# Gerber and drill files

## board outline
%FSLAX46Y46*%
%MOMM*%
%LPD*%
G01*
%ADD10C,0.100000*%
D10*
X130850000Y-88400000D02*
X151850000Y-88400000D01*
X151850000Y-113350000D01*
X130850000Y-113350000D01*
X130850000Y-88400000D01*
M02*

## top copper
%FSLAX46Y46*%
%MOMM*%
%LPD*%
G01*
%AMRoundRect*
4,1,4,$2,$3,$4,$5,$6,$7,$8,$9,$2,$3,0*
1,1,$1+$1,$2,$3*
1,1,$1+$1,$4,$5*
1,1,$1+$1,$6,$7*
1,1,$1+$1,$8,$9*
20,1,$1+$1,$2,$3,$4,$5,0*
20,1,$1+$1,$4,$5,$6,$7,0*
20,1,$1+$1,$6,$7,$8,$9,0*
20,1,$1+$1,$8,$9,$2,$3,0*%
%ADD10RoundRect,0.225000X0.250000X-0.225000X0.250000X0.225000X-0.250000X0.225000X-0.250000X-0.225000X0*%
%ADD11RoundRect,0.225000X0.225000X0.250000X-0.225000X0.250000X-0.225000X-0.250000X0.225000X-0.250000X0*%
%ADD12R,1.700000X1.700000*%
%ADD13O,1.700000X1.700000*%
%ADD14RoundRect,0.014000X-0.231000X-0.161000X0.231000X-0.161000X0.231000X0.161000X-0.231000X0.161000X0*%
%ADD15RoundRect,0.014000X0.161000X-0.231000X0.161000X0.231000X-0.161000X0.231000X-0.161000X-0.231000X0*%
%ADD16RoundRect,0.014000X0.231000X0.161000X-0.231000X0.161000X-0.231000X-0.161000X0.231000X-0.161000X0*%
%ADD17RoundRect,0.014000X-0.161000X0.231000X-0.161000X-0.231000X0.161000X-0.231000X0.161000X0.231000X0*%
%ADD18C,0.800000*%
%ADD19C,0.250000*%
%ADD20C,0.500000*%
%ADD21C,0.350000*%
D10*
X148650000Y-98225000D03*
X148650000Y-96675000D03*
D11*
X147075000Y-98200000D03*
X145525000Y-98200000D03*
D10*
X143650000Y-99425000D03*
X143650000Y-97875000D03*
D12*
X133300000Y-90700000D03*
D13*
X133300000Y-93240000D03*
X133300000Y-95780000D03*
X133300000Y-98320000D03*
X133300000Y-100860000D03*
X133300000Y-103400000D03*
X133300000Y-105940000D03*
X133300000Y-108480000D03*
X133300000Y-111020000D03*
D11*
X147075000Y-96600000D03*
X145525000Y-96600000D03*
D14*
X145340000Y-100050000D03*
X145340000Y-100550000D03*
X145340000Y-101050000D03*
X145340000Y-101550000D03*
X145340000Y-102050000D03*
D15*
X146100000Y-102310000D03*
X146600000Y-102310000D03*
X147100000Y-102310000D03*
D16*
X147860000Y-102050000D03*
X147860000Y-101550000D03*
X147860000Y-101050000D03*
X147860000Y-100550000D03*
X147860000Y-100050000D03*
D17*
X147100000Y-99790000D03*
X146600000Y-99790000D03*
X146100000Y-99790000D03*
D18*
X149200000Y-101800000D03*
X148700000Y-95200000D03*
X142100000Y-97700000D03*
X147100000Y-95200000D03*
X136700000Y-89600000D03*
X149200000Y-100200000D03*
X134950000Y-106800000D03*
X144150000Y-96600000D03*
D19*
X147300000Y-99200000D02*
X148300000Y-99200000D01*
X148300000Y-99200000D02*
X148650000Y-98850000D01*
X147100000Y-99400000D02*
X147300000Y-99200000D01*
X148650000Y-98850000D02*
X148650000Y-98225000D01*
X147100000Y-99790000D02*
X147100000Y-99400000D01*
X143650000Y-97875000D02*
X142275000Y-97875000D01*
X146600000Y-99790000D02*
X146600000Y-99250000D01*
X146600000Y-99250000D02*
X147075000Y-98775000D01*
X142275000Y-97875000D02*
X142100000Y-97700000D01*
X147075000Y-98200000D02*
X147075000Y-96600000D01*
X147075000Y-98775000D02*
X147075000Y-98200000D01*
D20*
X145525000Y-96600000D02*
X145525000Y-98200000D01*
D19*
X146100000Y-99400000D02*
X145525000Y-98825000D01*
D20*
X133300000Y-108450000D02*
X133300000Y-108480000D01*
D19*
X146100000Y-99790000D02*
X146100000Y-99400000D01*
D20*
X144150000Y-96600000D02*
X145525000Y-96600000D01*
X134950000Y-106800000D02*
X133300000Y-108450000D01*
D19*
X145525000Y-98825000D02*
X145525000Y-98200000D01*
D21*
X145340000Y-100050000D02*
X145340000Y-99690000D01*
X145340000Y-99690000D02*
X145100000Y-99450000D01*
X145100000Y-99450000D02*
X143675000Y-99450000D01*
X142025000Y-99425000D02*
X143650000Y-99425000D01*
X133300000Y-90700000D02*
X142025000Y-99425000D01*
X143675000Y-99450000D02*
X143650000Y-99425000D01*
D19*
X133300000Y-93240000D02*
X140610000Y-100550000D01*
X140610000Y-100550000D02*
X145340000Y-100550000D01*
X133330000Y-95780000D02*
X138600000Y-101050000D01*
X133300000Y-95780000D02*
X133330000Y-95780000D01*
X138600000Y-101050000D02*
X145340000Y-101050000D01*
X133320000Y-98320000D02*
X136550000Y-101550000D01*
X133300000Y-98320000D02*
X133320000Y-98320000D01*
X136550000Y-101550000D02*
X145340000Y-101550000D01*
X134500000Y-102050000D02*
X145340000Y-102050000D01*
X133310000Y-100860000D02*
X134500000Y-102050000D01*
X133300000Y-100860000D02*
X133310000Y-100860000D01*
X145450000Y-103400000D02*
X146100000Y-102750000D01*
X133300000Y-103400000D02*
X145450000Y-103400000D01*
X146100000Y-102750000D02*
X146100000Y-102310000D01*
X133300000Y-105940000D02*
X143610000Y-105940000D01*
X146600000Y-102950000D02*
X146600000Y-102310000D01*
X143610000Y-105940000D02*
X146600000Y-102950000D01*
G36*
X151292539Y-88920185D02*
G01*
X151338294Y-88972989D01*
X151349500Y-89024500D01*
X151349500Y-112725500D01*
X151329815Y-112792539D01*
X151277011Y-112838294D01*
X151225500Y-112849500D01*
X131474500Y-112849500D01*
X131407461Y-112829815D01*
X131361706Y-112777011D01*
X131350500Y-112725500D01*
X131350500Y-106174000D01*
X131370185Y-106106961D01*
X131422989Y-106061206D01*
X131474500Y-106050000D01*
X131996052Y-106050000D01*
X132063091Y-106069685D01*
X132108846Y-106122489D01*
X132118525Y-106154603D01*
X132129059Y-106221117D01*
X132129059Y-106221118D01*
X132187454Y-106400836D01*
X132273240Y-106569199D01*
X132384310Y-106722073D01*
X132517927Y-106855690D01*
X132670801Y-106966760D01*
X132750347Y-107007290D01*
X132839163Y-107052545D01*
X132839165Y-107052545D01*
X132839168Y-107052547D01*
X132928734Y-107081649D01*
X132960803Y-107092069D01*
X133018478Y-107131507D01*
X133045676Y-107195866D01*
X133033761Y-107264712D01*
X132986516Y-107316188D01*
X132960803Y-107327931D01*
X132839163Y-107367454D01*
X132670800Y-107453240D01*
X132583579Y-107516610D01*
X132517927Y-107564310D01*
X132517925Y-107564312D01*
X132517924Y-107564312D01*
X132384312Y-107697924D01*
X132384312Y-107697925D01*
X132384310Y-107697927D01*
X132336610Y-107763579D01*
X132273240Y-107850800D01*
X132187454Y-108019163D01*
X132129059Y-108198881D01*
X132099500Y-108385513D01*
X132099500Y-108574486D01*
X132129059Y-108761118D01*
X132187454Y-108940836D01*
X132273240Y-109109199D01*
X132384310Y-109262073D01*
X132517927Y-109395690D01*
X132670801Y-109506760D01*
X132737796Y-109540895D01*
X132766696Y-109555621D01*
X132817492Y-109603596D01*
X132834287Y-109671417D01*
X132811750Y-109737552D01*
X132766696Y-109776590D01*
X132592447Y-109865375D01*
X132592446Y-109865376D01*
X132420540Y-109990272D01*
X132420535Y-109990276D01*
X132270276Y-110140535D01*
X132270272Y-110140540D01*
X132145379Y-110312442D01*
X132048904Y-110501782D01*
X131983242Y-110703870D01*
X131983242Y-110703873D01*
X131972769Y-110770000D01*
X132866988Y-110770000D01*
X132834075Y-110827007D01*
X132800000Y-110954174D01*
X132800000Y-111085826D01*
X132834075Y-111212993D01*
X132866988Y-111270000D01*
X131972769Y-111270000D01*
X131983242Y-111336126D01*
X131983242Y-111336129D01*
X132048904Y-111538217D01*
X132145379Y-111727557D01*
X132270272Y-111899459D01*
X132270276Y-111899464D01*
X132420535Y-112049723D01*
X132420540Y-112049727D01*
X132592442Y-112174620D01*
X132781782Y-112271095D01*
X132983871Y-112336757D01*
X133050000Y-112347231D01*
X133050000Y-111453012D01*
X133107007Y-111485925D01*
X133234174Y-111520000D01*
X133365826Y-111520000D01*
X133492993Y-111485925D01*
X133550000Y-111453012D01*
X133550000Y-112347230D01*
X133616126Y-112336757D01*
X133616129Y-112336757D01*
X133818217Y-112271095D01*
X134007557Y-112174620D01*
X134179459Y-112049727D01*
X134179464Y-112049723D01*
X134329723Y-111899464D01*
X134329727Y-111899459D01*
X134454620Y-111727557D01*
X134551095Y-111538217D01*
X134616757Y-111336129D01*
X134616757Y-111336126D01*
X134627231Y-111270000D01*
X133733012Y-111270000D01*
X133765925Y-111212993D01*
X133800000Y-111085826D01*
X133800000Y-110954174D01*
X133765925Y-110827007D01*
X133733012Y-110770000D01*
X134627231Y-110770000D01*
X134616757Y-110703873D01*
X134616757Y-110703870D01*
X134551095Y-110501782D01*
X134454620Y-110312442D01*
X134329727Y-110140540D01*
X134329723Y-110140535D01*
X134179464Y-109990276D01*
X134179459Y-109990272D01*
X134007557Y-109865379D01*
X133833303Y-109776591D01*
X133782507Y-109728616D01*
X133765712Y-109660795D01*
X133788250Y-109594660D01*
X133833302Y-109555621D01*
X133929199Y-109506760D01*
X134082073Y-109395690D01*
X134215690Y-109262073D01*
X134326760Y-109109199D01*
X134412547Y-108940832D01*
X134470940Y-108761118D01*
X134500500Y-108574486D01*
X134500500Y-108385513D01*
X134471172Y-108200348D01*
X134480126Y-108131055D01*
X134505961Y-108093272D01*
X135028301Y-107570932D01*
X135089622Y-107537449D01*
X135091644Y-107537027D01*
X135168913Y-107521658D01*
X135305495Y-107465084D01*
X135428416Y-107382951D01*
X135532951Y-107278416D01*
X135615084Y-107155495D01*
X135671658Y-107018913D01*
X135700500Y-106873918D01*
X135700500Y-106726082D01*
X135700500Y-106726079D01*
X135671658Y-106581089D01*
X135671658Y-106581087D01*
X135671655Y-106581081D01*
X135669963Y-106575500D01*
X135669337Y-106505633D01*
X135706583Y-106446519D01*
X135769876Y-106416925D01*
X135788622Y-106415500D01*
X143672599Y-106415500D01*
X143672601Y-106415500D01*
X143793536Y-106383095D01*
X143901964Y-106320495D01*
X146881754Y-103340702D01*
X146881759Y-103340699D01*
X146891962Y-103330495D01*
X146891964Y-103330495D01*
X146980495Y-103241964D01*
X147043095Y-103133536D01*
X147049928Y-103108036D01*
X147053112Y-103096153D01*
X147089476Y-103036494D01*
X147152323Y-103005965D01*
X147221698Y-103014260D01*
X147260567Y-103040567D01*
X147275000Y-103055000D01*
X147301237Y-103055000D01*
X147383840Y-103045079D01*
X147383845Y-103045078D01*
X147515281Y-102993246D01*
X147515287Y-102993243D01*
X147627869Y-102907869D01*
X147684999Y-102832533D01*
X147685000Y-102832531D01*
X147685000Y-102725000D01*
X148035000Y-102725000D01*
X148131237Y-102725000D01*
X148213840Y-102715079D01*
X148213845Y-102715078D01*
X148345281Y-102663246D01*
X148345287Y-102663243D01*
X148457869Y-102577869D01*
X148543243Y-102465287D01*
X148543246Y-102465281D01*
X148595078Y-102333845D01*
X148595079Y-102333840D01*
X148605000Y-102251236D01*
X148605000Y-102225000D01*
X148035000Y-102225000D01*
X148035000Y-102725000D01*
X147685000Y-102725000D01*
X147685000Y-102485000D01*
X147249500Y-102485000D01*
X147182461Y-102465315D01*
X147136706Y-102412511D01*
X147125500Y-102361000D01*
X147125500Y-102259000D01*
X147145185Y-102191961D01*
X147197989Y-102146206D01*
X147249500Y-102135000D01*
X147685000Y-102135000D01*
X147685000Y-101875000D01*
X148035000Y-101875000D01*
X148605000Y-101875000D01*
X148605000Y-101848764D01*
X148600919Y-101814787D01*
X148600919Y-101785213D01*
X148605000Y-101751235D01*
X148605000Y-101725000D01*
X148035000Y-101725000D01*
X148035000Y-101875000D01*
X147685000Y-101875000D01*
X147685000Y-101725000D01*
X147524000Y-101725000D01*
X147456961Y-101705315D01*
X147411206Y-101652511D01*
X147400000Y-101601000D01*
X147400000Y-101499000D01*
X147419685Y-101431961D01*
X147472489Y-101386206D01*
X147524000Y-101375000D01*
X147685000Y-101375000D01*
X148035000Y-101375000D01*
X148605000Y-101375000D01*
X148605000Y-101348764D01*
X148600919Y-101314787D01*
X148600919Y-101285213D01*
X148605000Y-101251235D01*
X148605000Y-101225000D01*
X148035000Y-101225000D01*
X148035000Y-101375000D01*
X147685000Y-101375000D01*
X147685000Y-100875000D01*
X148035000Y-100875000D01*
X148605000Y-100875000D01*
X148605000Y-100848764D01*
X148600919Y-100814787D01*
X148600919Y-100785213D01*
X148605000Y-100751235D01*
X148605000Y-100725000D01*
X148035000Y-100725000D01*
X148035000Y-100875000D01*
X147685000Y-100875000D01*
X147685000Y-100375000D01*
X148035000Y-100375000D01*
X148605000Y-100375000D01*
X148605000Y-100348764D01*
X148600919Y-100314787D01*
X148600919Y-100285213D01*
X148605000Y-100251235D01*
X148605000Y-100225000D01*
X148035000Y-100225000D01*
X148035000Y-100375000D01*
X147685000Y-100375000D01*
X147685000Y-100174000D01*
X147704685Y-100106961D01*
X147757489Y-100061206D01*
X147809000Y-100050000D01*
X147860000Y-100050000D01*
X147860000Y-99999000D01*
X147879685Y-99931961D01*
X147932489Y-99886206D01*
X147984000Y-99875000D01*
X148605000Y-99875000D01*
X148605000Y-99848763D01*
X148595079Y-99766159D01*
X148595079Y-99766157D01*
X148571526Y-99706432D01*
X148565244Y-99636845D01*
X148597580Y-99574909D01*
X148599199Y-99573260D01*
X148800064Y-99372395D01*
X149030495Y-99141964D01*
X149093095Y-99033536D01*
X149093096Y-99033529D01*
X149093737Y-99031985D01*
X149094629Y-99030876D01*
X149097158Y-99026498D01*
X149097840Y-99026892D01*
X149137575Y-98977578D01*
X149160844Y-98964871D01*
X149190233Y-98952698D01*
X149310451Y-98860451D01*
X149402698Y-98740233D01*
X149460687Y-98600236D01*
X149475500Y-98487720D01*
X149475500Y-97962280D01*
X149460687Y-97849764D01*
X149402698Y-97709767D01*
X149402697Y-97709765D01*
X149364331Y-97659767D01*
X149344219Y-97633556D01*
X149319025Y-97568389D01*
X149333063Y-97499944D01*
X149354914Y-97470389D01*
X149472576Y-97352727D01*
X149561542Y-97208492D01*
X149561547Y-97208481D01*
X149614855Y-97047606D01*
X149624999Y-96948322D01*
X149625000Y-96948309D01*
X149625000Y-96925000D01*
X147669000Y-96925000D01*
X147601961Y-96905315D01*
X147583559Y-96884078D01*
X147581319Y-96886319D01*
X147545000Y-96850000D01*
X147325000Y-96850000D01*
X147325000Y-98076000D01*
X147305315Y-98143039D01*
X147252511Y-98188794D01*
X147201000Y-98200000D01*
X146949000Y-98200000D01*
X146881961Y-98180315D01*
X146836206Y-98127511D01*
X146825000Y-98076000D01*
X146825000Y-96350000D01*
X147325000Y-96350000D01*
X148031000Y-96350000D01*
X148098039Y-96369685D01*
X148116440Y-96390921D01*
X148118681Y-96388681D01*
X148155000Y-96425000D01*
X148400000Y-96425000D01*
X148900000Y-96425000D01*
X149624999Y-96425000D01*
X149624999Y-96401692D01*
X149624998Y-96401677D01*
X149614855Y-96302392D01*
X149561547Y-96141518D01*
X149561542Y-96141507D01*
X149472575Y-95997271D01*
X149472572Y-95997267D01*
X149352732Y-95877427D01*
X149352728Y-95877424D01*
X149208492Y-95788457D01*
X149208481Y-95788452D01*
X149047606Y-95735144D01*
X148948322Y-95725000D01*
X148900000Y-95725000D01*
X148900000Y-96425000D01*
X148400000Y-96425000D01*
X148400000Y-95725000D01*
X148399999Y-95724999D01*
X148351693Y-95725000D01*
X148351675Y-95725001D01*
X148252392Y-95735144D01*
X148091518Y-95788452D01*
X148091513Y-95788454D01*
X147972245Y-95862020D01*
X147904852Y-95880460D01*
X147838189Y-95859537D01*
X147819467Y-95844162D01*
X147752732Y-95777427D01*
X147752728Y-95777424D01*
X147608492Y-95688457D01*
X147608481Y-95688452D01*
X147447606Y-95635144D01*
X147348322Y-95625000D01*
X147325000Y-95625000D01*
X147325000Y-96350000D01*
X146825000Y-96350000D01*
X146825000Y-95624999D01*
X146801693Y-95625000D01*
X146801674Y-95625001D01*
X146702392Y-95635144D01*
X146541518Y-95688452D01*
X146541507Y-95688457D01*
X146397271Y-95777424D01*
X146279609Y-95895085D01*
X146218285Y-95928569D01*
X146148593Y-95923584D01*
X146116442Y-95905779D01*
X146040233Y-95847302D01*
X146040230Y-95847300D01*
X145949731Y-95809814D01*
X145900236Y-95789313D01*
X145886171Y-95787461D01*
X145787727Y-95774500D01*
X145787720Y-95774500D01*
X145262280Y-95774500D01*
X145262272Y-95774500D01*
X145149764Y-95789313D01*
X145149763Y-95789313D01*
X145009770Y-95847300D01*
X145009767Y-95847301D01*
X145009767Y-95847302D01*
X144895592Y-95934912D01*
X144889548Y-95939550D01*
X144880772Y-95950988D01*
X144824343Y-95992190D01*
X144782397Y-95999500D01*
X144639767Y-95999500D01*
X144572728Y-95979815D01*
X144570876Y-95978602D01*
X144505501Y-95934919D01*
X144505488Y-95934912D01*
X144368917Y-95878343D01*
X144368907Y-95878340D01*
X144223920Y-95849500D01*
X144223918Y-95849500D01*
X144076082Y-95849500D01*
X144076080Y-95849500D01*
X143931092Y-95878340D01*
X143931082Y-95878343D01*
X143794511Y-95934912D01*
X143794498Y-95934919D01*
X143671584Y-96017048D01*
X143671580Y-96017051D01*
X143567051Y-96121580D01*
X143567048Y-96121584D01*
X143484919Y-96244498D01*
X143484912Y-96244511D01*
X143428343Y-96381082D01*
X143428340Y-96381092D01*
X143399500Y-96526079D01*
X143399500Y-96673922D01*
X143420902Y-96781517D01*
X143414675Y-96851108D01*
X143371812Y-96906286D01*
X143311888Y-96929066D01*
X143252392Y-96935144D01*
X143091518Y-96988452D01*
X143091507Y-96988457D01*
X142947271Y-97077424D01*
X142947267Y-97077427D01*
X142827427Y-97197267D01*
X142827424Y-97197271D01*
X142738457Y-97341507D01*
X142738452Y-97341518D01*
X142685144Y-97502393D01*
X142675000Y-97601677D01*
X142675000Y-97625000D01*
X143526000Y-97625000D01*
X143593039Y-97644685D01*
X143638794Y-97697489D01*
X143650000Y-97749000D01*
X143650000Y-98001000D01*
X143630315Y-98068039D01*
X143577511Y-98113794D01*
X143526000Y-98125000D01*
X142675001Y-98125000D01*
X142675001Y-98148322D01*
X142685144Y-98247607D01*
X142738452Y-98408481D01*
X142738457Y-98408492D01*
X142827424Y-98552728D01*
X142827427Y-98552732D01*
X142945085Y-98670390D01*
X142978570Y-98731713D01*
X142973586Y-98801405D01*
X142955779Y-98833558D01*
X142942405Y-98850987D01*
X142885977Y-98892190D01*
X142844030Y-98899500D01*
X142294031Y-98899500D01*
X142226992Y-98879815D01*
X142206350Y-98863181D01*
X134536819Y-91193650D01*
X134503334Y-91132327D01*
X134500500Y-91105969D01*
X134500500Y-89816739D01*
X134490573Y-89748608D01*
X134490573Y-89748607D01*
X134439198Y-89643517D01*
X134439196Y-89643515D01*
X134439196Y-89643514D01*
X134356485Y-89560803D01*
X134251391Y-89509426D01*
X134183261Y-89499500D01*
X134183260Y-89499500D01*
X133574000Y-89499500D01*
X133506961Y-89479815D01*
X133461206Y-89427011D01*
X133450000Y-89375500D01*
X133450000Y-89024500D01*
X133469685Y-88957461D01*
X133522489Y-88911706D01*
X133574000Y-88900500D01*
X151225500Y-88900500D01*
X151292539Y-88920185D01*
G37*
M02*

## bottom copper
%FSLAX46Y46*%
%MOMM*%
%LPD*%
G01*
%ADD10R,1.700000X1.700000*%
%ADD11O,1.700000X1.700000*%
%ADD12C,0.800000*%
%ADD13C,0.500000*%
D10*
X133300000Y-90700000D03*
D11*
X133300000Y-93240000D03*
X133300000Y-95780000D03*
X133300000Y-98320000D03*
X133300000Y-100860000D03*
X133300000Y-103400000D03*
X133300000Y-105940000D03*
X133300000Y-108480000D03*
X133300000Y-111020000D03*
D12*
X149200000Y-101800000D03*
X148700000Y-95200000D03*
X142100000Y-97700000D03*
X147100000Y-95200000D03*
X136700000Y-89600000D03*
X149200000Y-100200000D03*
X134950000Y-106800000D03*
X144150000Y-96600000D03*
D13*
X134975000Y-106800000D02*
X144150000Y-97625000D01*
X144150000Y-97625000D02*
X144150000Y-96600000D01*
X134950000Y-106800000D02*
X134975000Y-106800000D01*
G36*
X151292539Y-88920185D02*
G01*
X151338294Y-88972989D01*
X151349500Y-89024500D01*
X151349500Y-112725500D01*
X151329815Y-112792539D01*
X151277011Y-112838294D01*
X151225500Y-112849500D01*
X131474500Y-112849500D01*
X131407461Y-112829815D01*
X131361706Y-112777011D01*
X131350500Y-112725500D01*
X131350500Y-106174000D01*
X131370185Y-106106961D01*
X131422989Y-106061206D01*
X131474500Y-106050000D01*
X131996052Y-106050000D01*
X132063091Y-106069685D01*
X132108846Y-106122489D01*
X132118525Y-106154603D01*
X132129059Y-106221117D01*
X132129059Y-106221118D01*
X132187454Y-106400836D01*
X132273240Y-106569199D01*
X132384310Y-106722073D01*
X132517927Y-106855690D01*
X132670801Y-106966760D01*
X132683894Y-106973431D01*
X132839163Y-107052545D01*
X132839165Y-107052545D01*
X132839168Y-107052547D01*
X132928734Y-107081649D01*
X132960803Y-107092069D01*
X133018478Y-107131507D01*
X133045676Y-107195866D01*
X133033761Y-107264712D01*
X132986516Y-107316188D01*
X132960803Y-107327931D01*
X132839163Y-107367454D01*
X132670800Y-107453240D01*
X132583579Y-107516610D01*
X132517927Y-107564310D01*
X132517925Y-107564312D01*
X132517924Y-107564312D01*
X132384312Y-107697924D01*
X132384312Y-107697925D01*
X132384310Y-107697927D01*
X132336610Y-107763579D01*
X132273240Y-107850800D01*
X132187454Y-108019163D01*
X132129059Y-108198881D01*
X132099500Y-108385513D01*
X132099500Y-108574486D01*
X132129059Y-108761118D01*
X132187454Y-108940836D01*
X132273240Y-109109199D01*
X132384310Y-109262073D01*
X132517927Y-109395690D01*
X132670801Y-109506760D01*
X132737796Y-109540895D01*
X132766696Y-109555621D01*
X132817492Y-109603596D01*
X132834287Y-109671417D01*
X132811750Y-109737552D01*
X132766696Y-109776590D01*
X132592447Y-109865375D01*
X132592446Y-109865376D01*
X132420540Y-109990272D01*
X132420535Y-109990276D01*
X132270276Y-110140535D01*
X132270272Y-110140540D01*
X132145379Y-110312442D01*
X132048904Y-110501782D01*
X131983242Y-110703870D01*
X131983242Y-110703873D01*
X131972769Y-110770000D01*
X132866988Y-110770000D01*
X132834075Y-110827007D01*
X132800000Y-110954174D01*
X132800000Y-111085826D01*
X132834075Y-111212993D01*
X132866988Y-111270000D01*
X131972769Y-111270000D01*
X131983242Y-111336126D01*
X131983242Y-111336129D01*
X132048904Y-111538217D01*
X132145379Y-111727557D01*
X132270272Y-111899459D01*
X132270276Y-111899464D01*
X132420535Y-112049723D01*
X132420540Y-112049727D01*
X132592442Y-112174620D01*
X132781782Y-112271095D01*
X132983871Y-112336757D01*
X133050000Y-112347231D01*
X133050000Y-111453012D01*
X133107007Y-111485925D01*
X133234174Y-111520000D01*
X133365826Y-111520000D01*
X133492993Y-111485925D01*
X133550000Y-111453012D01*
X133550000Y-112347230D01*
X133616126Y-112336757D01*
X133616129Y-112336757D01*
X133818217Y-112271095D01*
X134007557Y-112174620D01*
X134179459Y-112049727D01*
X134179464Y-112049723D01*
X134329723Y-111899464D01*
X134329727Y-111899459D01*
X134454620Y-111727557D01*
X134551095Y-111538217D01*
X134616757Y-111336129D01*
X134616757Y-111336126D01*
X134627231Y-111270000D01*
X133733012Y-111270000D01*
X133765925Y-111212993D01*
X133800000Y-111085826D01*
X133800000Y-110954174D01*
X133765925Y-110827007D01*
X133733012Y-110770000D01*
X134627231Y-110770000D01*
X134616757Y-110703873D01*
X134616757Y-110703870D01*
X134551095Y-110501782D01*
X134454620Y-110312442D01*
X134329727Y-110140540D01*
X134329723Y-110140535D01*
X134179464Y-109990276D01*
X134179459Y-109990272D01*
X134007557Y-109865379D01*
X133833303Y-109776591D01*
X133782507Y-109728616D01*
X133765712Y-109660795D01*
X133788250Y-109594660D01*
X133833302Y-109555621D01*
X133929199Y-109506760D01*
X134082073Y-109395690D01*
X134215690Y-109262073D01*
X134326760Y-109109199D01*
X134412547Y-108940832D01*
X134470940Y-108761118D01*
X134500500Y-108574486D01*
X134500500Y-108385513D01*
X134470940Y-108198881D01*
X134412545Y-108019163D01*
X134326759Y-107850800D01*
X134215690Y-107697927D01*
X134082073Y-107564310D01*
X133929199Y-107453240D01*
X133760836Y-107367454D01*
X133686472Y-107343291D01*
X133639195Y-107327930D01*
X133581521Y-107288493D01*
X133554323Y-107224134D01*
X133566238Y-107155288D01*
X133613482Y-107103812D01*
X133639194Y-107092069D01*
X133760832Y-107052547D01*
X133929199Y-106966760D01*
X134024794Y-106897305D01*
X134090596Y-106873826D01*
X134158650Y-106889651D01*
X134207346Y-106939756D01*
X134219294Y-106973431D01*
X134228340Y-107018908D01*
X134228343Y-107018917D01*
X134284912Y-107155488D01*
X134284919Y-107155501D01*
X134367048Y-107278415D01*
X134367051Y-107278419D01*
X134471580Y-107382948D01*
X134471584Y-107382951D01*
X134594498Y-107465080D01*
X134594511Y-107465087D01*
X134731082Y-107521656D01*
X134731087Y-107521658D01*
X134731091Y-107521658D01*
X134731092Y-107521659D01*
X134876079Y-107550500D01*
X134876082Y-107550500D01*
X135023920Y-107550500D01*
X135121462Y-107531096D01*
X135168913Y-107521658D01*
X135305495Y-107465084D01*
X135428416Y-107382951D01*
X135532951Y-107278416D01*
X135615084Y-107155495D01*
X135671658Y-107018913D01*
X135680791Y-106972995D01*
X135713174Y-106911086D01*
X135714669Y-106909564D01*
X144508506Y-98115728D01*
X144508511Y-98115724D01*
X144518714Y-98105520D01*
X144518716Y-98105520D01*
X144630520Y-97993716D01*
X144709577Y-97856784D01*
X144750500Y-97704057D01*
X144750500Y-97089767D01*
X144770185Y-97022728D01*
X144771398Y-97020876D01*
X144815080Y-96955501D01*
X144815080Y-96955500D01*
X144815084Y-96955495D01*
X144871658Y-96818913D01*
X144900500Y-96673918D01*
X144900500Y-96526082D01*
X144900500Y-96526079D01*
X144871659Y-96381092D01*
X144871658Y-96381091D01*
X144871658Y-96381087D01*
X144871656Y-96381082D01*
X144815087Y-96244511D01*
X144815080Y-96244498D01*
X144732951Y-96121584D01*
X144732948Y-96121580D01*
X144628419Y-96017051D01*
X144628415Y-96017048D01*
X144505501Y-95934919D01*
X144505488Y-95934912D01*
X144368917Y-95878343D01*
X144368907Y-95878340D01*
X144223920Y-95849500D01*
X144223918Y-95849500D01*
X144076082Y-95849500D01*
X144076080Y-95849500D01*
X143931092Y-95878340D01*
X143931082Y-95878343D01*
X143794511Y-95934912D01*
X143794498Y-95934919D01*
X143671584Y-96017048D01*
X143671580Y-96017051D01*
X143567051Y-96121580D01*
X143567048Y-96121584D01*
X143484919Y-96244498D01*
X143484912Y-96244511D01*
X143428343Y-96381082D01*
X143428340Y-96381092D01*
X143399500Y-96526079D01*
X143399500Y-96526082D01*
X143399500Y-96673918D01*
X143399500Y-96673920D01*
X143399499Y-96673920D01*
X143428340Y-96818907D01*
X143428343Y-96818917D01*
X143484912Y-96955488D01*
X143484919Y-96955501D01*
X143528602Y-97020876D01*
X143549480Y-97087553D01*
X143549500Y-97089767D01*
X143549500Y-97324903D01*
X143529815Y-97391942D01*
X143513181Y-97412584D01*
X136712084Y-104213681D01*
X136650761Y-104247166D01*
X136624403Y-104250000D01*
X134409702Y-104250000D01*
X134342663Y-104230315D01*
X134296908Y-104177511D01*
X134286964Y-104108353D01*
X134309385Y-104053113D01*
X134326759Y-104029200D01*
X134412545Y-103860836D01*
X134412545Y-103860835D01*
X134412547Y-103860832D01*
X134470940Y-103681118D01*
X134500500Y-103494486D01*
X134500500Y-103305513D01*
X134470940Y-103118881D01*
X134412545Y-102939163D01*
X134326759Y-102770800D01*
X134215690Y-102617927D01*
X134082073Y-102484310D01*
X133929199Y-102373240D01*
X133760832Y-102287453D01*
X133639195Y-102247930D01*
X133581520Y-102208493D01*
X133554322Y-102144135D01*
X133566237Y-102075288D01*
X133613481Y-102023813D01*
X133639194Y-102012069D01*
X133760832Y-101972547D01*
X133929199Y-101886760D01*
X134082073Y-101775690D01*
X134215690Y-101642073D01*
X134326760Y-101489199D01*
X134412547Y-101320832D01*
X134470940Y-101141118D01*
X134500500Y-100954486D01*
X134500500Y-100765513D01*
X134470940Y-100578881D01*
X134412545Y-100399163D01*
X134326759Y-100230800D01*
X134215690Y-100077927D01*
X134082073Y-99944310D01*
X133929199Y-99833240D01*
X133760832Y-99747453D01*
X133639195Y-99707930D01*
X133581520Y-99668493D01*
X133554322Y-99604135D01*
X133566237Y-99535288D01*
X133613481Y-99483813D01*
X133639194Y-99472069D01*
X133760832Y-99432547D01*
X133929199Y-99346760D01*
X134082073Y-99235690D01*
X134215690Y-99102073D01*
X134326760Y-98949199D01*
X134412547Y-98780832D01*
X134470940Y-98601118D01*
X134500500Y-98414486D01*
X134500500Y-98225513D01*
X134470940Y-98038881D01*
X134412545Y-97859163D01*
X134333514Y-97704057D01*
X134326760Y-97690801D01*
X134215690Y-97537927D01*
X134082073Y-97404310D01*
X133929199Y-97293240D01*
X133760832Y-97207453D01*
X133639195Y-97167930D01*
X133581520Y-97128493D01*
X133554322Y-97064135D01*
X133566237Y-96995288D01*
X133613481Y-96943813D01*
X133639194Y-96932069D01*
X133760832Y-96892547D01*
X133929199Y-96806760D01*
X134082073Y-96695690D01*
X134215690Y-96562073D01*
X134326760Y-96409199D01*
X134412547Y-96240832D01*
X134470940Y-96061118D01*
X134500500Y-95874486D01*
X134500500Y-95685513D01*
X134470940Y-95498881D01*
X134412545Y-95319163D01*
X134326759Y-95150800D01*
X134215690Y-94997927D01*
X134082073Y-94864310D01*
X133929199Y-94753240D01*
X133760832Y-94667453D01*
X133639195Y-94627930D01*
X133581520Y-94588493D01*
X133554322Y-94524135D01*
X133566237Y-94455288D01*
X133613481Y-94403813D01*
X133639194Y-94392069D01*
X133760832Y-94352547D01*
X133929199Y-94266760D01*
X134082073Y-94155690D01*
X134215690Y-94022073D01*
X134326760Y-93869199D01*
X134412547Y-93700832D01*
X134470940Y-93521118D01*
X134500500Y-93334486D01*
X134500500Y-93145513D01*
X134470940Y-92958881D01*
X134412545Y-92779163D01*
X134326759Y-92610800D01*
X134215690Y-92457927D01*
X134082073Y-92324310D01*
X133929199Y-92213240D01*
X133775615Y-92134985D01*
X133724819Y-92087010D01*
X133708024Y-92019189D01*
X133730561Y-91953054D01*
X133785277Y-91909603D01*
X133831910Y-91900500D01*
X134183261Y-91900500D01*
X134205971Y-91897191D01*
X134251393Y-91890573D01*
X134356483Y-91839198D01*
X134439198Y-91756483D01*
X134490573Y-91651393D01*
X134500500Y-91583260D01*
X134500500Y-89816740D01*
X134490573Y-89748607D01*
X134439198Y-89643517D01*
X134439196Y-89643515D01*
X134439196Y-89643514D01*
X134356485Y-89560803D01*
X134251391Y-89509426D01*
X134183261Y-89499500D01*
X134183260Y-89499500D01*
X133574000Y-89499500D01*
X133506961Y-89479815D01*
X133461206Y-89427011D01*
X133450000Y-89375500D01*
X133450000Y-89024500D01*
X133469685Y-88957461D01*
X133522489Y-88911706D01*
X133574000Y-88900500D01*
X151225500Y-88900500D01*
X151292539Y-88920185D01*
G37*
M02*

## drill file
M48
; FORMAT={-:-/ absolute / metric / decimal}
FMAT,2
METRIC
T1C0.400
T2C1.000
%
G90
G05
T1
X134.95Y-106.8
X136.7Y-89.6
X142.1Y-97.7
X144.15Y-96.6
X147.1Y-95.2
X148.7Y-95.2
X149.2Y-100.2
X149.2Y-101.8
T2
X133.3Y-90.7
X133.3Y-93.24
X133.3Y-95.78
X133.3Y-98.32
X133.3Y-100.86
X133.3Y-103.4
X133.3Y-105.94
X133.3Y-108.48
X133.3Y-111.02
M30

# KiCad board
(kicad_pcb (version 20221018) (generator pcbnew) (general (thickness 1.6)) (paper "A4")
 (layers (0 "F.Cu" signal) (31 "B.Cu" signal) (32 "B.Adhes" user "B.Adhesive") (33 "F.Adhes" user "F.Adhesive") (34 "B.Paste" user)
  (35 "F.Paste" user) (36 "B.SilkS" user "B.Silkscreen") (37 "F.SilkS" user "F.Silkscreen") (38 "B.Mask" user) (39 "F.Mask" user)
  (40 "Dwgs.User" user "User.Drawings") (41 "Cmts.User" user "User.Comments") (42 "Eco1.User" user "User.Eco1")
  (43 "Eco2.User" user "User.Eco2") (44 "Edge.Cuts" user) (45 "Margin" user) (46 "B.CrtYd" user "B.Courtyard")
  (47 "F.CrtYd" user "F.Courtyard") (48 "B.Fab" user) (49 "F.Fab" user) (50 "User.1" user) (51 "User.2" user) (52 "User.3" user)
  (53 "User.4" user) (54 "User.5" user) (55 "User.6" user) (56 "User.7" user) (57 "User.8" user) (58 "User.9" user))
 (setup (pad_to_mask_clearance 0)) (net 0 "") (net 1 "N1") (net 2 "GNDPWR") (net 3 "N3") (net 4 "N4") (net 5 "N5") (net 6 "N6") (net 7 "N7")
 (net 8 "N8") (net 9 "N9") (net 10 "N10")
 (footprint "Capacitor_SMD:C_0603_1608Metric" (layer "F.Cu") (at 148.65 97.45 90)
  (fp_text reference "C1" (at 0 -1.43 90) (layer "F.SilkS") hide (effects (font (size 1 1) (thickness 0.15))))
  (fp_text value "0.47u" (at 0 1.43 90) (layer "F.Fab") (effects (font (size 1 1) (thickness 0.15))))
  (pad "1" smd roundrect (at -0.775 0 90) (size 0.9 0.95) (layers "F.Cu" "F.Paste" "F.Mask") (roundrect_rratio 0.25) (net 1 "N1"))
  (pad "2" smd roundrect (at 0.775 0 90) (size 0.9 0.95) (layers "F.Cu" "F.Paste" "F.Mask") (roundrect_rratio 0.25) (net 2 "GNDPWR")))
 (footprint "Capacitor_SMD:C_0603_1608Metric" (layer "F.Cu") (at 146.3 98.2 180)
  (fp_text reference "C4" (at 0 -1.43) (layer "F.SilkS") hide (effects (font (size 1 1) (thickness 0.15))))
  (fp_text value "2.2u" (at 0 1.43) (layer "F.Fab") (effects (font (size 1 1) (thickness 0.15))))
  (pad "1" smd roundrect (at -0.775 0 180) (size 0.9 0.95) (layers "F.Cu" "F.Paste" "F.Mask") (roundrect_rratio 0.25) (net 2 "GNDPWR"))
  (pad "2" smd roundrect (at 0.775 0 180) (size 0.9 0.95) (layers "F.Cu" "F.Paste" "F.Mask") (roundrect_rratio 0.25) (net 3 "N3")))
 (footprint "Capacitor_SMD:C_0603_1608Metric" (layer "F.Cu") (at 143.65 98.65 90)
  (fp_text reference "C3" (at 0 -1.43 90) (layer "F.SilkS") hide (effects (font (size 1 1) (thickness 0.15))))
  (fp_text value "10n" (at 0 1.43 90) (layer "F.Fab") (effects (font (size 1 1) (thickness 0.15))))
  (pad "1" smd roundrect (at -0.775 0 90) (size 0.9 0.95) (layers "F.Cu" "F.Paste" "F.Mask") (roundrect_rratio 0.25) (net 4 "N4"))
  (pad "2" smd roundrect (at 0.775 0 90) (size 0.9 0.95) (layers "F.Cu" "F.Paste" "F.Mask") (roundrect_rratio 0.25) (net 2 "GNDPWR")))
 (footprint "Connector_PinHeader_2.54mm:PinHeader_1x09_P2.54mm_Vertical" (layer "F.Cu") (at 133.3 90.7)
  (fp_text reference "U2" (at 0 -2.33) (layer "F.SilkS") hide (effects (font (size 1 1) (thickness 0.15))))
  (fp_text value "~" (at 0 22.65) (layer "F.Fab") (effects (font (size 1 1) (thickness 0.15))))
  (pad "1" thru_hole rect (at 0 0) (size 1.7 1.7) (drill 1) (layers "*.Cu" "*.Mask") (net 4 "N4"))
  (pad "2" thru_hole oval (at 0 2.54) (size 1.7 1.7) (drill 1) (layers "*.Cu" "*.Mask") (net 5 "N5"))
  (pad "3" thru_hole oval (at 0 5.08) (size 1.7 1.7) (drill 1) (layers "*.Cu" "*.Mask") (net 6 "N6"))
  (pad "4" thru_hole oval (at 0 7.62) (size 1.7 1.7) (drill 1) (layers "*.Cu" "*.Mask") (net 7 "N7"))
  (pad "5" thru_hole oval (at 0 10.16) (size 1.7 1.7) (drill 1) (layers "*.Cu" "*.Mask") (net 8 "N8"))
  (pad "6" thru_hole oval (at 0 12.7) (size 1.7 1.7) (drill 1) (layers "*.Cu" "*.Mask") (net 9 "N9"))
  (pad "7" thru_hole oval (at 0 15.24) (size 1.7 1.7) (drill 1) (layers "*.Cu" "*.Mask") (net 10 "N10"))
  (pad "8" thru_hole oval (at 0 17.78) (size 1.7 1.7) (drill 1) (layers "*.Cu" "*.Mask") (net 3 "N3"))
  (pad "9" thru_hole oval (at 0 20.32) (size 1.7 1.7) (drill 1) (layers "*.Cu" "*.Mask") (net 2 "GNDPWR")))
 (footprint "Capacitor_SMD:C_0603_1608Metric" (layer "F.Cu") (at 146.3 96.6 180)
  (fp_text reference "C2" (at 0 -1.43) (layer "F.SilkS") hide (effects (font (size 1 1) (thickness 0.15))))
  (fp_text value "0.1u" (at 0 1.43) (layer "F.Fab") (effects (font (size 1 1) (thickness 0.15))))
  (pad "1" smd roundrect (at -0.775 0 180) (size 0.9 0.95) (layers "F.Cu" "F.Paste" "F.Mask") (roundrect_rratio 0.25) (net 2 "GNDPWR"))
  (pad "2" smd roundrect (at 0.775 0 180) (size 0.9 0.95) (layers "F.Cu" "F.Paste" "F.Mask") (roundrect_rratio 0.25) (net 3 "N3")))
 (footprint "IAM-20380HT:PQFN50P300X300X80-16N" (layer "F.Cu") (at 146.6 101.05)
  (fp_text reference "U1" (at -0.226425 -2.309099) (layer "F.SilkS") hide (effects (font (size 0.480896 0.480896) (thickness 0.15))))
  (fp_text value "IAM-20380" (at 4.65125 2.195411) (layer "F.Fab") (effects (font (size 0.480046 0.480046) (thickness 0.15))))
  (pad "1" smd roundrect (at -1.26 -1) (size 0.49 0.35) (layers "F.Cu" "F.Paste" "F.Mask") (roundrect_rratio 0.04) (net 4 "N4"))
  (pad "2" smd roundrect (at -1.26 -0.5) (size 0.49 0.35) (layers "F.Cu" "F.Paste" "F.Mask") (roundrect_rratio 0.04) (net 5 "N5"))
  (pad "3" smd roundrect (at -1.26 0) (size 0.49 0.35) (layers "F.Cu" "F.Paste" "F.Mask") (roundrect_rratio 0.04) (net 6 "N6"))
  (pad "4" smd roundrect (at -1.26 0.5) (size 0.49 0.35) (layers "F.Cu" "F.Paste" "F.Mask") (roundrect_rratio 0.04) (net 7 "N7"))
  (pad "5" smd roundrect (at -1.26 1) (size 0.49 0.35) (layers "F.Cu" "F.Paste" "F.Mask") (roundrect_rratio 0.04) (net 8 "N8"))
  (pad "6" smd roundrect (at -0.5 1.26 90) (size 0.49 0.35) (layers "F.Cu" "F.Paste" "F.Mask") (roundrect_rratio 0.04) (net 9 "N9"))
  (pad "7" smd roundrect (at 0 1.26 90) (size 0.49 0.35) (layers "F.Cu" "F.Paste" "F.Mask") (roundrect_rratio 0.04) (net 10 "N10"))
  (pad "8" smd roundrect (at 0.5 1.26 90) (size 0.49 0.35) (layers "F.Cu" "F.Paste" "F.Mask") (roundrect_rratio 0.04) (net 2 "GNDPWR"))
  (pad "9" smd roundrect (at 1.26 1 180) (size 0.49 0.35) (layers "F.Cu" "F.Paste" "F.Mask") (roundrect_rratio 0.04) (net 2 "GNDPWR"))
  (pad "10" smd roundrect (at 1.26 0.5 180) (size 0.49 0.35) (layers "F.Cu" "F.Paste" "F.Mask") (roundrect_rratio 0.04) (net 2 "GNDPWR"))
  (pad "11" smd roundrect (at 1.26 0 180) (size 0.49 0.35) (layers "F.Cu" "F.Paste" "F.Mask") (roundrect_rratio 0.04) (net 2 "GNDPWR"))
  (pad "12" smd roundrect (at 1.26 -0.5 180) (size 0.49 0.35) (layers "F.Cu" "F.Paste" "F.Mask") (roundrect_rratio 0.04) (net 2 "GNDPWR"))
  (pad "13" smd roundrect (at 1.26 -1 180) (size 0.49 0.35) (layers "F.Cu" "F.Paste" "F.Mask") (roundrect_rratio 0.04) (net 2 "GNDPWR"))
  (pad "14" smd roundrect (at 0.5 -1.26 270) (size 0.49 0.35) (layers "F.Cu" "F.Paste" "F.Mask") (roundrect_rratio 0.04) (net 1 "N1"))
  (pad "15" smd roundrect (at 0 -1.26 270) (size 0.49 0.35) (layers "F.Cu" "F.Paste" "F.Mask") (roundrect_rratio 0.04) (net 2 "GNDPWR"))
  (pad "16" smd roundrect (at -0.5 -1.26 270) (size 0.49 0.35) (layers "F.Cu" "F.Paste" "F.Mask") (roundrect_rratio 0.04) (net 3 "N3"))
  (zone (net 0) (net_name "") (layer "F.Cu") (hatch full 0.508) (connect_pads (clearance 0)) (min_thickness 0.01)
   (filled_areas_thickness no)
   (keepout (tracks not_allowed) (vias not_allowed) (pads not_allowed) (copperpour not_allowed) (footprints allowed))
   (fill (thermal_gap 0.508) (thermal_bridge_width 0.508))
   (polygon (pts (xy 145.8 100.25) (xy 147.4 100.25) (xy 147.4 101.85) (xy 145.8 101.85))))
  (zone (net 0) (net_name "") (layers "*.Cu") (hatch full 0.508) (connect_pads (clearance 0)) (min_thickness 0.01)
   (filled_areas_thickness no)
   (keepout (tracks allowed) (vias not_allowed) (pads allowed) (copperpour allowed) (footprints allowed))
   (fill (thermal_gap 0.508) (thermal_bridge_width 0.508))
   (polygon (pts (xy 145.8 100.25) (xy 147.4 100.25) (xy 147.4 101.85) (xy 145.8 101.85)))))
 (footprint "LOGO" (layer "B.Cu") (at 146.6 108 180)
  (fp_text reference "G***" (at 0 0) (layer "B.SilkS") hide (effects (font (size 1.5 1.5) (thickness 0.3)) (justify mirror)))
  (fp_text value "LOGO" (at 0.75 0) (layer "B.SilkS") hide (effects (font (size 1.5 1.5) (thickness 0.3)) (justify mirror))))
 (gr_rect (start 130.85 88.4) (end 151.85 113.35) (stroke (width 0.1) (type default)) (fill none) (layer "Edge.Cuts"))
 (segment (start 147.3 99.2) (end 148.3 99.2) (width 0.25) (layer "F.Cu") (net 1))
 (segment (start 148.3 99.2) (end 148.65 98.85) (width 0.25) (layer "F.Cu") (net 1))
 (segment (start 147.1 99.4) (end 147.3 99.2) (width 0.25) (layer "F.Cu") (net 1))
 (segment (start 148.65 98.85) (end 148.65 98.225) (width 0.25) (layer "F.Cu") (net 1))
 (segment (start 147.1 99.79) (end 147.1 99.4) (width 0.25) (layer "F.Cu") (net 1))
 (segment (start 143.65 97.875) (end 142.275 97.875) (width 0.25) (layer "F.Cu") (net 2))
 (segment (start 146.6 99.79) (end 146.6 99.25) (width 0.25) (layer "F.Cu") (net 2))
 (segment (start 146.6 99.25) (end 147.075 98.775) (width 0.25) (layer "F.Cu") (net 2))
 (segment (start 142.275 97.875) (end 142.1 97.7) (width 0.25) (layer "F.Cu") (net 2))
 (segment (start 147.075 98.2) (end 147.075 96.6) (width 0.25) (layer "F.Cu") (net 2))
 (segment (start 147.075 98.775) (end 147.075 98.2) (width 0.25) (layer "F.Cu") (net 2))
 (via (at 149.2 101.8) (size 0.8) (drill 0.4) (layers "F.Cu" "B.Cu") (free) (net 2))
 (via (at 148.7 95.2) (size 0.8) (drill 0.4) (layers "F.Cu" "B.Cu") (free) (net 2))
 (via (at 142.1 97.7) (size 0.8) (drill 0.4) (layers "F.Cu" "B.Cu") (free) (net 2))
 (via (at 147.1 95.2) (size 0.8) (drill 0.4) (layers "F.Cu" "B.Cu") (free) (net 2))
 (via (at 136.7 89.6) (size 0.8) (drill 0.4) (layers "F.Cu" "B.Cu") (free) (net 2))
 (via (at 149.2 100.2) (size 0.8) (drill 0.4) (layers "F.Cu" "B.Cu") (free) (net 2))
 (segment (start 145.525 96.6) (end 145.525 98.2) (width 0.5) (layer "F.Cu") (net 3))
 (segment (start 146.1 99.4) (end 145.525 98.825) (width 0.25) (layer "F.Cu") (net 3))
 (segment (start 133.3 108.45) (end 133.3 108.48) (width 0.5) (layer "F.Cu") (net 3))
 (segment (start 146.1 99.79) (end 146.1 99.4) (width 0.25) (layer "F.Cu") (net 3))
 (segment (start 144.15 96.6) (end 145.525 96.6) (width 0.5) (layer "F.Cu") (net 3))
 (segment (start 134.95 106.8) (end 133.3 108.45) (width 0.5) (layer "F.Cu") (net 3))
 (segment (start 145.525 98.825) (end 145.525 98.2) (width 0.25) (layer "F.Cu") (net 3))
 (via (at 134.95 106.8) (size 0.8) (drill 0.4) (layers "F.Cu" "B.Cu") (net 3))
 (via (at 144.15 96.6) (size 0.8) (drill 0.4) (layers "F.Cu" "B.Cu") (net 3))
 (segment (start 134.975 106.8) (end 144.15 97.625) (width 0.5) (layer "B.Cu") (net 3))
 (segment (start 144.15 97.625) (end 144.15 96.6) (width 0.5) (layer "B.Cu") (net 3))
 (segment (start 134.95 106.8) (end 134.975 106.8) (width 0.5) (layer "B.Cu") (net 3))
 (segment (start 145.34 100.05) (end 145.34 99.69) (width 0.35) (layer "F.Cu") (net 4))
 (segment (start 145.34 99.69) (end 145.1 99.45) (width 0.35) (layer "F.Cu") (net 4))
 (segment (start 145.1 99.45) (end 143.675 99.45) (width 0.35) (layer "F.Cu") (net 4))
 (segment (start 142.025 99.425) (end 143.65 99.425) (width 0.35) (layer "F.Cu") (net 4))
 (segment (start 133.3 90.7) (end 142.025 99.425) (width 0.35) (layer "F.Cu") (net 4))
 (segment (start 143.675 99.45) (end 143.65 99.425) (width 0.35) (layer "F.Cu") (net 4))
 (segment (start 133.3 93.24) (end 140.61 100.55) (width 0.25) (layer "F.Cu") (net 5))
 (segment (start 140.61 100.55) (end 145.34 100.55) (width 0.25) (layer "F.Cu") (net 5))
 (segment (start 133.33 95.78) (end 138.6 101.05) (width 0.25) (layer "F.Cu") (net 6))
 (segment (start 133.3 95.78) (end 133.33 95.78) (width 0.25) (layer "F.Cu") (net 6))
 (segment (start 138.6 101.05) (end 145.34 101.05) (width 0.25) (layer "F.Cu") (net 6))
 (segment (start 133.32 98.32) (end 136.55 101.55) (width 0.25) (layer "F.Cu") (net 7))
 (segment (start 133.3 98.32) (end 133.32 98.32) (width 0.25) (layer "F.Cu") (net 7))
 (segment (start 136.55 101.55) (end 145.34 101.55) (width 0.25) (layer "F.Cu") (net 7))
 (segment (start 134.5 102.05) (end 145.34 102.05) (width 0.25) (layer "F.Cu") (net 8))
 (segment (start 133.31 100.86) (end 134.5 102.05) (width 0.25) (layer "F.Cu") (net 8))
 (segment (start 133.3 100.86) (end 133.31 100.86) (width 0.25) (layer "F.Cu") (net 8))
 (segment (start 145.45 103.4) (end 146.1 102.75) (width 0.25) (layer "F.Cu") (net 9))
 (segment (start 133.3 103.4) (end 145.45 103.4) (width 0.25) (layer "F.Cu") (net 9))
 (segment (start 146.1 102.75) (end 146.1 102.31) (width 0.25) (layer "F.Cu") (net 9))
 (segment (start 133.3 105.94) (end 143.61 105.94) (width 0.25) (layer "F.Cu") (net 10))
 (segment (start 146.6 102.95) (end 146.6 102.31) (width 0.25) (layer "F.Cu") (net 10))
 (segment (start 143.61 105.94) (end 146.6 102.95) (width 0.25) (layer "F.Cu") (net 10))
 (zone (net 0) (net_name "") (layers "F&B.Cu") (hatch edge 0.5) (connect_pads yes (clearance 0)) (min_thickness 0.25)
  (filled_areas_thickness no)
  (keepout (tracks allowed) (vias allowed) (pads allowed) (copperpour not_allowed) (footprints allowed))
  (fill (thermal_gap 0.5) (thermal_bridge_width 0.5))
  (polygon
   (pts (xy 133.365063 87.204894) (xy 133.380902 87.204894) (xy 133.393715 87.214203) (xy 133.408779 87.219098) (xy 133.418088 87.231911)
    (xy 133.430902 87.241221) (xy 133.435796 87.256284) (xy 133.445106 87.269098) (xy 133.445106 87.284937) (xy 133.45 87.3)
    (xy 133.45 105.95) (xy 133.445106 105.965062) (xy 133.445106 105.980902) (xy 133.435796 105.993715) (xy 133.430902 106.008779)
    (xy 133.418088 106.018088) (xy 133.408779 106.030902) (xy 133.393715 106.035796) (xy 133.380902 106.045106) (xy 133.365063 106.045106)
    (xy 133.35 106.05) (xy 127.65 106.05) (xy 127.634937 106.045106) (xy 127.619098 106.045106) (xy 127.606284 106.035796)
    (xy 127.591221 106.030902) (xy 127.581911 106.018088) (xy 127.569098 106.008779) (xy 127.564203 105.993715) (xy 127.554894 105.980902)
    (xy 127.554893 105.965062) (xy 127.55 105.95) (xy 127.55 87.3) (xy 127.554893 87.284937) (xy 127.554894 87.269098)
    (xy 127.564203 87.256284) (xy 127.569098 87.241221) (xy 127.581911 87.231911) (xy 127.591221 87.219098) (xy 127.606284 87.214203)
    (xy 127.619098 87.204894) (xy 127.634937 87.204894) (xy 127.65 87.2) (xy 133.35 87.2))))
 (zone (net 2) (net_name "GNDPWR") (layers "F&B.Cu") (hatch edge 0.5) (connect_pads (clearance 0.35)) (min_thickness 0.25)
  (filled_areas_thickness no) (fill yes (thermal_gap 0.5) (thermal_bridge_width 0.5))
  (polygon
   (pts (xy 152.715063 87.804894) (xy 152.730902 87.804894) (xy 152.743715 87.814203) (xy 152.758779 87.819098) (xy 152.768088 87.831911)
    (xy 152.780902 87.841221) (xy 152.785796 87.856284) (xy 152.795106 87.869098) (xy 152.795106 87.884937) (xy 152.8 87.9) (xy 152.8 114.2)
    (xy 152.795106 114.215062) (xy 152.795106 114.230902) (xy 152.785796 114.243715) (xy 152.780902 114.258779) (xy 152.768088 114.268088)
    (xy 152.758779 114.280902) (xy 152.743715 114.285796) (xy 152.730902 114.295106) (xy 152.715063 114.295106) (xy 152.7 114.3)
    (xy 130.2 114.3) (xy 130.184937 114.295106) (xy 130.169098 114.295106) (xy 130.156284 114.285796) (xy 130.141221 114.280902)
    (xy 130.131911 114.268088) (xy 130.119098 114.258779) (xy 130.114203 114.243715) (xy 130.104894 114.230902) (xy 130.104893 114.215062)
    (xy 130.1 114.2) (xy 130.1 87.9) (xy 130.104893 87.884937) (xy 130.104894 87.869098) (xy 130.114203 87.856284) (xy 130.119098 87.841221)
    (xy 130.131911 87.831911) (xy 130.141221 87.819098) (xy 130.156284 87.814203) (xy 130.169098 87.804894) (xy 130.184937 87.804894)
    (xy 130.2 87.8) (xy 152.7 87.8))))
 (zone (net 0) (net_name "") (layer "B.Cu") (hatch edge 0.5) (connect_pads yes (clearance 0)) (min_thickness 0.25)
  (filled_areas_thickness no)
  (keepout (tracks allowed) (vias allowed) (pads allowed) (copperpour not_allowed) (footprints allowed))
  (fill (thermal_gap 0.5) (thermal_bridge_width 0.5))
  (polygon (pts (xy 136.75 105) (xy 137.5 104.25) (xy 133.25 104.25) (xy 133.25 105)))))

